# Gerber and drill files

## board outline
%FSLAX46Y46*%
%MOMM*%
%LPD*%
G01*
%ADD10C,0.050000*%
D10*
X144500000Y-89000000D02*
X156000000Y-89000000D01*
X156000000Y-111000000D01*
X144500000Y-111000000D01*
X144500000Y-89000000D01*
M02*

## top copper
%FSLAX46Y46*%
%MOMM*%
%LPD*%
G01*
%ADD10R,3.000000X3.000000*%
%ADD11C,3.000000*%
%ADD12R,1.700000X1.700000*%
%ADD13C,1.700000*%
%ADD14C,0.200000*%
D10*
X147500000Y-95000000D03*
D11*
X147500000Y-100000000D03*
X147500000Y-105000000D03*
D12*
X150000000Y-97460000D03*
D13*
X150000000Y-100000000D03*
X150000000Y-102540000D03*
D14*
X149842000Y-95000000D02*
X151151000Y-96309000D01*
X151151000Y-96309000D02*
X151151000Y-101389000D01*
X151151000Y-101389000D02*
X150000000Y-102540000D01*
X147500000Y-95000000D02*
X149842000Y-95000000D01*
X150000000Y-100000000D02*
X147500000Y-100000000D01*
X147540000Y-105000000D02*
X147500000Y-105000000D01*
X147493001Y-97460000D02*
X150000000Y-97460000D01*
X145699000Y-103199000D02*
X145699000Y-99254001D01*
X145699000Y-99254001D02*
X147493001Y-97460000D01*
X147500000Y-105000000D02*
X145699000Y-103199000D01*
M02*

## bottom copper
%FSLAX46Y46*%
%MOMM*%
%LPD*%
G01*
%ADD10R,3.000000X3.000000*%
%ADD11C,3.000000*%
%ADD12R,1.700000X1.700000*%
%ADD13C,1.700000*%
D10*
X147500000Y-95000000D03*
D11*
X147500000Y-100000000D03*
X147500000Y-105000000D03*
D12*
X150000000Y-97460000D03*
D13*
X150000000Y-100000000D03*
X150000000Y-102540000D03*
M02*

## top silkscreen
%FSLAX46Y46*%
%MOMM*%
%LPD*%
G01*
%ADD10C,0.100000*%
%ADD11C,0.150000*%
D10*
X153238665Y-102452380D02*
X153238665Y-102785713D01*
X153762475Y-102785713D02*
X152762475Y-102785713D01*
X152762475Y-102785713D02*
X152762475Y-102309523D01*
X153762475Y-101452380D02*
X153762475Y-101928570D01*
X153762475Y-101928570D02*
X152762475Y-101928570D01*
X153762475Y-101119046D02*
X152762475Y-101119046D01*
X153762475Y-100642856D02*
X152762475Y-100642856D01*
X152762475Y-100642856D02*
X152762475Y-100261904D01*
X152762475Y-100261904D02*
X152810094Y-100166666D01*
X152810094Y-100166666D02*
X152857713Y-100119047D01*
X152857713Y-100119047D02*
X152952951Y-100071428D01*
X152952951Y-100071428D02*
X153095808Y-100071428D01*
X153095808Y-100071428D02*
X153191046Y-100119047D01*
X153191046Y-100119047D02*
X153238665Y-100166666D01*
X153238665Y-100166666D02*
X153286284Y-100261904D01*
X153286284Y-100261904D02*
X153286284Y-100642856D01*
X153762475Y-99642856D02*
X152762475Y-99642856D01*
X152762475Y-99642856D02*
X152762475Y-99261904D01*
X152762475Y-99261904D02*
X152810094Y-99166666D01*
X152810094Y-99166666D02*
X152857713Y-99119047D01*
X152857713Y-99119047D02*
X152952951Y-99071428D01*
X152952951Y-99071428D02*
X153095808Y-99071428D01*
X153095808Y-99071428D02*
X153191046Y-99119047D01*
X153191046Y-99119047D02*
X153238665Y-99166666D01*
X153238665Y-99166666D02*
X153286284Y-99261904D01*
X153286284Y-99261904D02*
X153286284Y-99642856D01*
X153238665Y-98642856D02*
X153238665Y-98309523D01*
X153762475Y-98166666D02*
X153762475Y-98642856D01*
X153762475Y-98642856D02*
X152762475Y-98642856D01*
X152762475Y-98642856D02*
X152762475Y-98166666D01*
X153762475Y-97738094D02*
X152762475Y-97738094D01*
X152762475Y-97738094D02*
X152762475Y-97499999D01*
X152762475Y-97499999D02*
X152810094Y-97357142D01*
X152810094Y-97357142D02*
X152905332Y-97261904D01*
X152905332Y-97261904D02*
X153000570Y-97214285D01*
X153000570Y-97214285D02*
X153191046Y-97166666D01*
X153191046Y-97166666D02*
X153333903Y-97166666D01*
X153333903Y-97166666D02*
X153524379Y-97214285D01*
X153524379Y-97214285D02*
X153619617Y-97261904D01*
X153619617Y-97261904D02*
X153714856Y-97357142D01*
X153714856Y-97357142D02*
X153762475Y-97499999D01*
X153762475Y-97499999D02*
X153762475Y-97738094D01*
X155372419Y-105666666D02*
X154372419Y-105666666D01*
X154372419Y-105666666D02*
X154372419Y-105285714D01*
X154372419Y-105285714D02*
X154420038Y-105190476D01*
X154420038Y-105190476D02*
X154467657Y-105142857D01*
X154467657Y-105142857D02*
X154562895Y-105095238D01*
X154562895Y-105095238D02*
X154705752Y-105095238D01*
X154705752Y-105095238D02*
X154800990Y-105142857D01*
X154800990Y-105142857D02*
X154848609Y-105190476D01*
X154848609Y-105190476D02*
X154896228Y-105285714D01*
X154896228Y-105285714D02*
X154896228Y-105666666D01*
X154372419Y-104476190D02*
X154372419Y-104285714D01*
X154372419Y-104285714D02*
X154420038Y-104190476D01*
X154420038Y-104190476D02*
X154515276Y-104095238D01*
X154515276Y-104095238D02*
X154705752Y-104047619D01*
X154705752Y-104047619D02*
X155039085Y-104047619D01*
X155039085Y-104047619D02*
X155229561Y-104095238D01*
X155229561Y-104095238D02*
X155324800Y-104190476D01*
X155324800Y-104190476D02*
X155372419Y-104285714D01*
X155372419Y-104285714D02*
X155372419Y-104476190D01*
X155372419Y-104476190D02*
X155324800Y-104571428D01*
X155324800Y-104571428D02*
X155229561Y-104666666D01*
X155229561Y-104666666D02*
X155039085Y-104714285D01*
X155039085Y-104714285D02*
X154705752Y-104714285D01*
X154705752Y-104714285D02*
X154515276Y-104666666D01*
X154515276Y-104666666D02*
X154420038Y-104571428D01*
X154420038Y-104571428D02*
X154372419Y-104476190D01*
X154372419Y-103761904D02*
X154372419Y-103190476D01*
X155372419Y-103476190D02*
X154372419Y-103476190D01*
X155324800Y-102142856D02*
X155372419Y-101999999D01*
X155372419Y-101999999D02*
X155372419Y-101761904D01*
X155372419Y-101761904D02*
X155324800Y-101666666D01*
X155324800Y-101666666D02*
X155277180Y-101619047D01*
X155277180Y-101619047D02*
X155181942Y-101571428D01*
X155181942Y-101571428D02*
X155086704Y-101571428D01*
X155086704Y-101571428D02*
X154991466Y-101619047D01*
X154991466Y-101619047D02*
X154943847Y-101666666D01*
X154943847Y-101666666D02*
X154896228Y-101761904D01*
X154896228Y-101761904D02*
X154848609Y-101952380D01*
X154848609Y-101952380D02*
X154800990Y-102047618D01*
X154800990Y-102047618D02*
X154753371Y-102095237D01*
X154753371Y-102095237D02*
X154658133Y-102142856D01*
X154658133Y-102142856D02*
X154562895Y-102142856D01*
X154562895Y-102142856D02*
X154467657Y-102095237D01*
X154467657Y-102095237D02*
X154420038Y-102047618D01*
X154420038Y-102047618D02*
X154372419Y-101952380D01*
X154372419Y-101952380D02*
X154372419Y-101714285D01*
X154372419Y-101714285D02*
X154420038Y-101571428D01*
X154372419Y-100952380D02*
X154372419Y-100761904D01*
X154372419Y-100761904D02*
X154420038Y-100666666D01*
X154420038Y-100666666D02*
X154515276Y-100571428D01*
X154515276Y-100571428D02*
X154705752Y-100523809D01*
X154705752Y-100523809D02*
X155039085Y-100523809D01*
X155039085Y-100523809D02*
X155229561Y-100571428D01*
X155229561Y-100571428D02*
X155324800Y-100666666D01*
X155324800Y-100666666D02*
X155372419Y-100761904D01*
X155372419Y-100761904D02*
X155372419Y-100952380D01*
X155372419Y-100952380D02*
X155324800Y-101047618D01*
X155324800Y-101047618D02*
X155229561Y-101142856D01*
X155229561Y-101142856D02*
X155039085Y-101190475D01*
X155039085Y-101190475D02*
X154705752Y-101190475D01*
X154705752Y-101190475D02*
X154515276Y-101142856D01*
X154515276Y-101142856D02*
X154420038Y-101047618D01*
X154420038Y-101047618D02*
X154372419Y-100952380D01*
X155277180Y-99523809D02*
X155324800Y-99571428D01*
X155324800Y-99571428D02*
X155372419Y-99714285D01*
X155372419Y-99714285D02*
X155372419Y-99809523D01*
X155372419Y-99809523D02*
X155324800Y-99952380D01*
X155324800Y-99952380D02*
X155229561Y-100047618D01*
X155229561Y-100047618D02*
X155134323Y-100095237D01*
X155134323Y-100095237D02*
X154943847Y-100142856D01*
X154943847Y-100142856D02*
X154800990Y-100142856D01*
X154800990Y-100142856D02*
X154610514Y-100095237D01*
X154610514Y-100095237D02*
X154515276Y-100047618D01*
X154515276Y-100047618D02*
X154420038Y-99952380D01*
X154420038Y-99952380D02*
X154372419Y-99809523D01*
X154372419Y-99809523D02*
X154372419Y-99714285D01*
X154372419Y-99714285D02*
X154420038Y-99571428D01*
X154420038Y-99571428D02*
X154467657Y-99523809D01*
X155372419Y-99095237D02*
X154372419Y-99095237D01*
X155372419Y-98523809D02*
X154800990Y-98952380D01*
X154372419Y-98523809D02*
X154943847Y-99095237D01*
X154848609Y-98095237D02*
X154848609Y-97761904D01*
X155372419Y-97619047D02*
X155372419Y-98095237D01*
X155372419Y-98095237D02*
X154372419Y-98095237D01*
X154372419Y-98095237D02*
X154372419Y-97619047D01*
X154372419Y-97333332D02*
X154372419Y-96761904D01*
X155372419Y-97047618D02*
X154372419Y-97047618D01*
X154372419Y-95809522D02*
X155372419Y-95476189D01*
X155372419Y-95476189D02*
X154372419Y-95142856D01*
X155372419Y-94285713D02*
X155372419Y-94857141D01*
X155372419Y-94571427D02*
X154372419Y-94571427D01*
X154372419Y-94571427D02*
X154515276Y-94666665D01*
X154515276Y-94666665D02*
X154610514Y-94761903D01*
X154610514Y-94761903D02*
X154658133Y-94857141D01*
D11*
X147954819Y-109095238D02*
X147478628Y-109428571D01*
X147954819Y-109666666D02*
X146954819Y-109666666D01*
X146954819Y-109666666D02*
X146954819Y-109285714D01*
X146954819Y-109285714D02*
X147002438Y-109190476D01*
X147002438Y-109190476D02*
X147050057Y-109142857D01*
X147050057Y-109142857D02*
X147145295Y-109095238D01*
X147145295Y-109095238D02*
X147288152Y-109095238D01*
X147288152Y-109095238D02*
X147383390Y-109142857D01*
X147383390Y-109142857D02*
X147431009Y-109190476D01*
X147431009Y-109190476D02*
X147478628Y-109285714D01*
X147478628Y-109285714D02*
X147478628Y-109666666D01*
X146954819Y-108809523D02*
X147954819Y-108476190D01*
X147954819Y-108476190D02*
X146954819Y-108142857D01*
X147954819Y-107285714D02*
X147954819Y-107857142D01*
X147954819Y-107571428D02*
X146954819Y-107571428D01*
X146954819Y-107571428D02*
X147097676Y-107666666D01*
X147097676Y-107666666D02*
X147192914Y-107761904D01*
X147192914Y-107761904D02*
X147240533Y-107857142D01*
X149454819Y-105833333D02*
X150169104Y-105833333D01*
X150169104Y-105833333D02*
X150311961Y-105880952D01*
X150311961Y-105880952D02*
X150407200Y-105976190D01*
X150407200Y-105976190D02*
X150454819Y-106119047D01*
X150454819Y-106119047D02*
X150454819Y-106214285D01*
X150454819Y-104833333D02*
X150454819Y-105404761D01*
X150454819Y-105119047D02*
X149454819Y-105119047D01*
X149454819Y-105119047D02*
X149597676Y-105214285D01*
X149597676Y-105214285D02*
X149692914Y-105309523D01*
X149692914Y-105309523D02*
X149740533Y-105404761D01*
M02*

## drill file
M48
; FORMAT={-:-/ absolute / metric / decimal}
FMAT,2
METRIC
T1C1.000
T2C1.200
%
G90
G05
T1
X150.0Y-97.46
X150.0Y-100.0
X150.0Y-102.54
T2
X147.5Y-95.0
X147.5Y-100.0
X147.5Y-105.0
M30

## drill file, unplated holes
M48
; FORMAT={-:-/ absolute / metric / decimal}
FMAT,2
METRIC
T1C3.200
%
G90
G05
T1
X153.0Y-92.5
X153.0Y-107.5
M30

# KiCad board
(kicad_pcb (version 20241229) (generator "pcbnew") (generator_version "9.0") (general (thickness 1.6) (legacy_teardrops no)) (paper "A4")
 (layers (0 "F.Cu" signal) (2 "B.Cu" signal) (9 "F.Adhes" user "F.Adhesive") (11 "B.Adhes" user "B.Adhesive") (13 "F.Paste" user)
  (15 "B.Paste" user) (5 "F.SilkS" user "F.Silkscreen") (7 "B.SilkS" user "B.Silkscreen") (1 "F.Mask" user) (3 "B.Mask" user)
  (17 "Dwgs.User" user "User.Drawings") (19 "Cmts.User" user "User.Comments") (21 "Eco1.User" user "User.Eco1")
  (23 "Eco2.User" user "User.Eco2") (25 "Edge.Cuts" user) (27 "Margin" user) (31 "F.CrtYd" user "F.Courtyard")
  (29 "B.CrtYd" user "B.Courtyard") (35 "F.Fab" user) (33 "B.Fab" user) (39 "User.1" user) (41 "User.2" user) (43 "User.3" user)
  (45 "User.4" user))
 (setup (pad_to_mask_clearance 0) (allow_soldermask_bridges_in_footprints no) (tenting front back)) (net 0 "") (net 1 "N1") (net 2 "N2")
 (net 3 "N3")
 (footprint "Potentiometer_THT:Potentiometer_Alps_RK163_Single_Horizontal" (layer "F.Cu") (at 147.5 95)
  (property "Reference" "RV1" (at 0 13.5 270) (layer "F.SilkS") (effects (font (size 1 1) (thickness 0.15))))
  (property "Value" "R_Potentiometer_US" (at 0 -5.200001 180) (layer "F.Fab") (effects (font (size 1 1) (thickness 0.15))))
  (pad "1" thru_hole rect (at 0 0 180) (size 3 3) (drill 1.2) (layers "*.Cu" "*.Mask") (remove_unused_layers no) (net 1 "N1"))
  (pad "2" thru_hole circle (at 0 5 180) (size 3 3) (drill 1.2) (layers "*.Cu" "*.Mask") (remove_unused_layers no) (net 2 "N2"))
  (pad "3" thru_hole circle (at 0 10 180) (size 3 3) (drill 1.2) (layers "*.Cu" "*.Mask") (remove_unused_layers no) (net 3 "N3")))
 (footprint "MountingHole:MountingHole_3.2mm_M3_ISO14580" (layer "F.Cu") (at 153 107.5)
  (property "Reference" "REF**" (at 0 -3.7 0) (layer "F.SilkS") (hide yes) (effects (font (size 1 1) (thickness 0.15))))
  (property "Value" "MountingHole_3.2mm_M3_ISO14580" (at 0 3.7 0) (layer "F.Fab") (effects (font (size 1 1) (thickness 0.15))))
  (pad "" np_thru_hole circle (at 0 0) (size 3.2 3.2) (drill 3.2) (layers "*.Cu" "*.Mask")))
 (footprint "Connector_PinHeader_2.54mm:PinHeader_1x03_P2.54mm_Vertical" (layer "F.Cu") (at 150 97.46)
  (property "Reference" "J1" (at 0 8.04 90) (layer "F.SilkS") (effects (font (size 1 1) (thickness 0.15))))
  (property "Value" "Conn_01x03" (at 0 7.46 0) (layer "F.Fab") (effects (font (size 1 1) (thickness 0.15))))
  (pad "1" thru_hole rect (at 0 0) (size 1.7 1.7) (drill 1) (layers "*.Cu" "*.Mask") (remove_unused_layers no) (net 3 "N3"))
  (pad "2" thru_hole circle (at 0 2.54) (size 1.7 1.7) (drill 1) (layers "*.Cu" "*.Mask") (remove_unused_layers no) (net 2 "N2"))
  (pad "3" thru_hole circle (at 0 5.08) (size 1.7 1.7) (drill 1) (layers "*.Cu" "*.Mask") (remove_unused_layers no) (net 1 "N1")))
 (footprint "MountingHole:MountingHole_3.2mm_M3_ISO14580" (layer "F.Cu") (at 153 92.5)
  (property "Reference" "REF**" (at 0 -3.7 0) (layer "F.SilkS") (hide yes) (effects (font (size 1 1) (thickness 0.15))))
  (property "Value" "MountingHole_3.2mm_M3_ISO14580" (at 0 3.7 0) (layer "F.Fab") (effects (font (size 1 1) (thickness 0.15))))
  (pad "" np_thru_hole circle (at 0 0) (size 3.2 3.2) (drill 3.2) (layers "*.Cu" "*.Mask")))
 (gr_rect (start 144.5 89) (end 156 111) (stroke (width 0.05) (type default)) (fill no) (layer "Edge.Cuts"))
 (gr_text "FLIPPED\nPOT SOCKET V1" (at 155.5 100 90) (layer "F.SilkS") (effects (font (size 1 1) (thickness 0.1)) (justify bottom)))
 (segment (start 149.842 95) (end 151.151 96.309) (width 0.2) (layer "F.Cu") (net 1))
 (segment (start 151.151 96.309) (end 151.151 101.389) (width 0.2) (layer "F.Cu") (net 1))
 (segment (start 151.151 101.389) (end 150 102.54) (width 0.2) (layer "F.Cu") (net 1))
 (segment (start 147.5 95) (end 149.842 95) (width 0.2) (layer "F.Cu") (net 1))
 (segment (start 150 100) (end 147.5 100) (width 0.2) (layer "F.Cu") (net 2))
 (segment (start 147.54 105) (end 147.5 105) (width 0.2) (layer "F.Cu") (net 3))
 (segment (start 147.493001 97.46) (end 150 97.46) (width 0.2) (layer "F.Cu") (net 3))
 (segment (start 145.699 103.199) (end 145.699 99.254001) (width 0.2) (layer "F.Cu") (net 3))
 (segment (start 145.699 99.254001) (end 147.493001 97.46) (width 0.2) (layer "F.Cu") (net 3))
 (segment (start 147.5 105) (end 145.699 103.199) (width 0.2) (layer "F.Cu") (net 3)))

